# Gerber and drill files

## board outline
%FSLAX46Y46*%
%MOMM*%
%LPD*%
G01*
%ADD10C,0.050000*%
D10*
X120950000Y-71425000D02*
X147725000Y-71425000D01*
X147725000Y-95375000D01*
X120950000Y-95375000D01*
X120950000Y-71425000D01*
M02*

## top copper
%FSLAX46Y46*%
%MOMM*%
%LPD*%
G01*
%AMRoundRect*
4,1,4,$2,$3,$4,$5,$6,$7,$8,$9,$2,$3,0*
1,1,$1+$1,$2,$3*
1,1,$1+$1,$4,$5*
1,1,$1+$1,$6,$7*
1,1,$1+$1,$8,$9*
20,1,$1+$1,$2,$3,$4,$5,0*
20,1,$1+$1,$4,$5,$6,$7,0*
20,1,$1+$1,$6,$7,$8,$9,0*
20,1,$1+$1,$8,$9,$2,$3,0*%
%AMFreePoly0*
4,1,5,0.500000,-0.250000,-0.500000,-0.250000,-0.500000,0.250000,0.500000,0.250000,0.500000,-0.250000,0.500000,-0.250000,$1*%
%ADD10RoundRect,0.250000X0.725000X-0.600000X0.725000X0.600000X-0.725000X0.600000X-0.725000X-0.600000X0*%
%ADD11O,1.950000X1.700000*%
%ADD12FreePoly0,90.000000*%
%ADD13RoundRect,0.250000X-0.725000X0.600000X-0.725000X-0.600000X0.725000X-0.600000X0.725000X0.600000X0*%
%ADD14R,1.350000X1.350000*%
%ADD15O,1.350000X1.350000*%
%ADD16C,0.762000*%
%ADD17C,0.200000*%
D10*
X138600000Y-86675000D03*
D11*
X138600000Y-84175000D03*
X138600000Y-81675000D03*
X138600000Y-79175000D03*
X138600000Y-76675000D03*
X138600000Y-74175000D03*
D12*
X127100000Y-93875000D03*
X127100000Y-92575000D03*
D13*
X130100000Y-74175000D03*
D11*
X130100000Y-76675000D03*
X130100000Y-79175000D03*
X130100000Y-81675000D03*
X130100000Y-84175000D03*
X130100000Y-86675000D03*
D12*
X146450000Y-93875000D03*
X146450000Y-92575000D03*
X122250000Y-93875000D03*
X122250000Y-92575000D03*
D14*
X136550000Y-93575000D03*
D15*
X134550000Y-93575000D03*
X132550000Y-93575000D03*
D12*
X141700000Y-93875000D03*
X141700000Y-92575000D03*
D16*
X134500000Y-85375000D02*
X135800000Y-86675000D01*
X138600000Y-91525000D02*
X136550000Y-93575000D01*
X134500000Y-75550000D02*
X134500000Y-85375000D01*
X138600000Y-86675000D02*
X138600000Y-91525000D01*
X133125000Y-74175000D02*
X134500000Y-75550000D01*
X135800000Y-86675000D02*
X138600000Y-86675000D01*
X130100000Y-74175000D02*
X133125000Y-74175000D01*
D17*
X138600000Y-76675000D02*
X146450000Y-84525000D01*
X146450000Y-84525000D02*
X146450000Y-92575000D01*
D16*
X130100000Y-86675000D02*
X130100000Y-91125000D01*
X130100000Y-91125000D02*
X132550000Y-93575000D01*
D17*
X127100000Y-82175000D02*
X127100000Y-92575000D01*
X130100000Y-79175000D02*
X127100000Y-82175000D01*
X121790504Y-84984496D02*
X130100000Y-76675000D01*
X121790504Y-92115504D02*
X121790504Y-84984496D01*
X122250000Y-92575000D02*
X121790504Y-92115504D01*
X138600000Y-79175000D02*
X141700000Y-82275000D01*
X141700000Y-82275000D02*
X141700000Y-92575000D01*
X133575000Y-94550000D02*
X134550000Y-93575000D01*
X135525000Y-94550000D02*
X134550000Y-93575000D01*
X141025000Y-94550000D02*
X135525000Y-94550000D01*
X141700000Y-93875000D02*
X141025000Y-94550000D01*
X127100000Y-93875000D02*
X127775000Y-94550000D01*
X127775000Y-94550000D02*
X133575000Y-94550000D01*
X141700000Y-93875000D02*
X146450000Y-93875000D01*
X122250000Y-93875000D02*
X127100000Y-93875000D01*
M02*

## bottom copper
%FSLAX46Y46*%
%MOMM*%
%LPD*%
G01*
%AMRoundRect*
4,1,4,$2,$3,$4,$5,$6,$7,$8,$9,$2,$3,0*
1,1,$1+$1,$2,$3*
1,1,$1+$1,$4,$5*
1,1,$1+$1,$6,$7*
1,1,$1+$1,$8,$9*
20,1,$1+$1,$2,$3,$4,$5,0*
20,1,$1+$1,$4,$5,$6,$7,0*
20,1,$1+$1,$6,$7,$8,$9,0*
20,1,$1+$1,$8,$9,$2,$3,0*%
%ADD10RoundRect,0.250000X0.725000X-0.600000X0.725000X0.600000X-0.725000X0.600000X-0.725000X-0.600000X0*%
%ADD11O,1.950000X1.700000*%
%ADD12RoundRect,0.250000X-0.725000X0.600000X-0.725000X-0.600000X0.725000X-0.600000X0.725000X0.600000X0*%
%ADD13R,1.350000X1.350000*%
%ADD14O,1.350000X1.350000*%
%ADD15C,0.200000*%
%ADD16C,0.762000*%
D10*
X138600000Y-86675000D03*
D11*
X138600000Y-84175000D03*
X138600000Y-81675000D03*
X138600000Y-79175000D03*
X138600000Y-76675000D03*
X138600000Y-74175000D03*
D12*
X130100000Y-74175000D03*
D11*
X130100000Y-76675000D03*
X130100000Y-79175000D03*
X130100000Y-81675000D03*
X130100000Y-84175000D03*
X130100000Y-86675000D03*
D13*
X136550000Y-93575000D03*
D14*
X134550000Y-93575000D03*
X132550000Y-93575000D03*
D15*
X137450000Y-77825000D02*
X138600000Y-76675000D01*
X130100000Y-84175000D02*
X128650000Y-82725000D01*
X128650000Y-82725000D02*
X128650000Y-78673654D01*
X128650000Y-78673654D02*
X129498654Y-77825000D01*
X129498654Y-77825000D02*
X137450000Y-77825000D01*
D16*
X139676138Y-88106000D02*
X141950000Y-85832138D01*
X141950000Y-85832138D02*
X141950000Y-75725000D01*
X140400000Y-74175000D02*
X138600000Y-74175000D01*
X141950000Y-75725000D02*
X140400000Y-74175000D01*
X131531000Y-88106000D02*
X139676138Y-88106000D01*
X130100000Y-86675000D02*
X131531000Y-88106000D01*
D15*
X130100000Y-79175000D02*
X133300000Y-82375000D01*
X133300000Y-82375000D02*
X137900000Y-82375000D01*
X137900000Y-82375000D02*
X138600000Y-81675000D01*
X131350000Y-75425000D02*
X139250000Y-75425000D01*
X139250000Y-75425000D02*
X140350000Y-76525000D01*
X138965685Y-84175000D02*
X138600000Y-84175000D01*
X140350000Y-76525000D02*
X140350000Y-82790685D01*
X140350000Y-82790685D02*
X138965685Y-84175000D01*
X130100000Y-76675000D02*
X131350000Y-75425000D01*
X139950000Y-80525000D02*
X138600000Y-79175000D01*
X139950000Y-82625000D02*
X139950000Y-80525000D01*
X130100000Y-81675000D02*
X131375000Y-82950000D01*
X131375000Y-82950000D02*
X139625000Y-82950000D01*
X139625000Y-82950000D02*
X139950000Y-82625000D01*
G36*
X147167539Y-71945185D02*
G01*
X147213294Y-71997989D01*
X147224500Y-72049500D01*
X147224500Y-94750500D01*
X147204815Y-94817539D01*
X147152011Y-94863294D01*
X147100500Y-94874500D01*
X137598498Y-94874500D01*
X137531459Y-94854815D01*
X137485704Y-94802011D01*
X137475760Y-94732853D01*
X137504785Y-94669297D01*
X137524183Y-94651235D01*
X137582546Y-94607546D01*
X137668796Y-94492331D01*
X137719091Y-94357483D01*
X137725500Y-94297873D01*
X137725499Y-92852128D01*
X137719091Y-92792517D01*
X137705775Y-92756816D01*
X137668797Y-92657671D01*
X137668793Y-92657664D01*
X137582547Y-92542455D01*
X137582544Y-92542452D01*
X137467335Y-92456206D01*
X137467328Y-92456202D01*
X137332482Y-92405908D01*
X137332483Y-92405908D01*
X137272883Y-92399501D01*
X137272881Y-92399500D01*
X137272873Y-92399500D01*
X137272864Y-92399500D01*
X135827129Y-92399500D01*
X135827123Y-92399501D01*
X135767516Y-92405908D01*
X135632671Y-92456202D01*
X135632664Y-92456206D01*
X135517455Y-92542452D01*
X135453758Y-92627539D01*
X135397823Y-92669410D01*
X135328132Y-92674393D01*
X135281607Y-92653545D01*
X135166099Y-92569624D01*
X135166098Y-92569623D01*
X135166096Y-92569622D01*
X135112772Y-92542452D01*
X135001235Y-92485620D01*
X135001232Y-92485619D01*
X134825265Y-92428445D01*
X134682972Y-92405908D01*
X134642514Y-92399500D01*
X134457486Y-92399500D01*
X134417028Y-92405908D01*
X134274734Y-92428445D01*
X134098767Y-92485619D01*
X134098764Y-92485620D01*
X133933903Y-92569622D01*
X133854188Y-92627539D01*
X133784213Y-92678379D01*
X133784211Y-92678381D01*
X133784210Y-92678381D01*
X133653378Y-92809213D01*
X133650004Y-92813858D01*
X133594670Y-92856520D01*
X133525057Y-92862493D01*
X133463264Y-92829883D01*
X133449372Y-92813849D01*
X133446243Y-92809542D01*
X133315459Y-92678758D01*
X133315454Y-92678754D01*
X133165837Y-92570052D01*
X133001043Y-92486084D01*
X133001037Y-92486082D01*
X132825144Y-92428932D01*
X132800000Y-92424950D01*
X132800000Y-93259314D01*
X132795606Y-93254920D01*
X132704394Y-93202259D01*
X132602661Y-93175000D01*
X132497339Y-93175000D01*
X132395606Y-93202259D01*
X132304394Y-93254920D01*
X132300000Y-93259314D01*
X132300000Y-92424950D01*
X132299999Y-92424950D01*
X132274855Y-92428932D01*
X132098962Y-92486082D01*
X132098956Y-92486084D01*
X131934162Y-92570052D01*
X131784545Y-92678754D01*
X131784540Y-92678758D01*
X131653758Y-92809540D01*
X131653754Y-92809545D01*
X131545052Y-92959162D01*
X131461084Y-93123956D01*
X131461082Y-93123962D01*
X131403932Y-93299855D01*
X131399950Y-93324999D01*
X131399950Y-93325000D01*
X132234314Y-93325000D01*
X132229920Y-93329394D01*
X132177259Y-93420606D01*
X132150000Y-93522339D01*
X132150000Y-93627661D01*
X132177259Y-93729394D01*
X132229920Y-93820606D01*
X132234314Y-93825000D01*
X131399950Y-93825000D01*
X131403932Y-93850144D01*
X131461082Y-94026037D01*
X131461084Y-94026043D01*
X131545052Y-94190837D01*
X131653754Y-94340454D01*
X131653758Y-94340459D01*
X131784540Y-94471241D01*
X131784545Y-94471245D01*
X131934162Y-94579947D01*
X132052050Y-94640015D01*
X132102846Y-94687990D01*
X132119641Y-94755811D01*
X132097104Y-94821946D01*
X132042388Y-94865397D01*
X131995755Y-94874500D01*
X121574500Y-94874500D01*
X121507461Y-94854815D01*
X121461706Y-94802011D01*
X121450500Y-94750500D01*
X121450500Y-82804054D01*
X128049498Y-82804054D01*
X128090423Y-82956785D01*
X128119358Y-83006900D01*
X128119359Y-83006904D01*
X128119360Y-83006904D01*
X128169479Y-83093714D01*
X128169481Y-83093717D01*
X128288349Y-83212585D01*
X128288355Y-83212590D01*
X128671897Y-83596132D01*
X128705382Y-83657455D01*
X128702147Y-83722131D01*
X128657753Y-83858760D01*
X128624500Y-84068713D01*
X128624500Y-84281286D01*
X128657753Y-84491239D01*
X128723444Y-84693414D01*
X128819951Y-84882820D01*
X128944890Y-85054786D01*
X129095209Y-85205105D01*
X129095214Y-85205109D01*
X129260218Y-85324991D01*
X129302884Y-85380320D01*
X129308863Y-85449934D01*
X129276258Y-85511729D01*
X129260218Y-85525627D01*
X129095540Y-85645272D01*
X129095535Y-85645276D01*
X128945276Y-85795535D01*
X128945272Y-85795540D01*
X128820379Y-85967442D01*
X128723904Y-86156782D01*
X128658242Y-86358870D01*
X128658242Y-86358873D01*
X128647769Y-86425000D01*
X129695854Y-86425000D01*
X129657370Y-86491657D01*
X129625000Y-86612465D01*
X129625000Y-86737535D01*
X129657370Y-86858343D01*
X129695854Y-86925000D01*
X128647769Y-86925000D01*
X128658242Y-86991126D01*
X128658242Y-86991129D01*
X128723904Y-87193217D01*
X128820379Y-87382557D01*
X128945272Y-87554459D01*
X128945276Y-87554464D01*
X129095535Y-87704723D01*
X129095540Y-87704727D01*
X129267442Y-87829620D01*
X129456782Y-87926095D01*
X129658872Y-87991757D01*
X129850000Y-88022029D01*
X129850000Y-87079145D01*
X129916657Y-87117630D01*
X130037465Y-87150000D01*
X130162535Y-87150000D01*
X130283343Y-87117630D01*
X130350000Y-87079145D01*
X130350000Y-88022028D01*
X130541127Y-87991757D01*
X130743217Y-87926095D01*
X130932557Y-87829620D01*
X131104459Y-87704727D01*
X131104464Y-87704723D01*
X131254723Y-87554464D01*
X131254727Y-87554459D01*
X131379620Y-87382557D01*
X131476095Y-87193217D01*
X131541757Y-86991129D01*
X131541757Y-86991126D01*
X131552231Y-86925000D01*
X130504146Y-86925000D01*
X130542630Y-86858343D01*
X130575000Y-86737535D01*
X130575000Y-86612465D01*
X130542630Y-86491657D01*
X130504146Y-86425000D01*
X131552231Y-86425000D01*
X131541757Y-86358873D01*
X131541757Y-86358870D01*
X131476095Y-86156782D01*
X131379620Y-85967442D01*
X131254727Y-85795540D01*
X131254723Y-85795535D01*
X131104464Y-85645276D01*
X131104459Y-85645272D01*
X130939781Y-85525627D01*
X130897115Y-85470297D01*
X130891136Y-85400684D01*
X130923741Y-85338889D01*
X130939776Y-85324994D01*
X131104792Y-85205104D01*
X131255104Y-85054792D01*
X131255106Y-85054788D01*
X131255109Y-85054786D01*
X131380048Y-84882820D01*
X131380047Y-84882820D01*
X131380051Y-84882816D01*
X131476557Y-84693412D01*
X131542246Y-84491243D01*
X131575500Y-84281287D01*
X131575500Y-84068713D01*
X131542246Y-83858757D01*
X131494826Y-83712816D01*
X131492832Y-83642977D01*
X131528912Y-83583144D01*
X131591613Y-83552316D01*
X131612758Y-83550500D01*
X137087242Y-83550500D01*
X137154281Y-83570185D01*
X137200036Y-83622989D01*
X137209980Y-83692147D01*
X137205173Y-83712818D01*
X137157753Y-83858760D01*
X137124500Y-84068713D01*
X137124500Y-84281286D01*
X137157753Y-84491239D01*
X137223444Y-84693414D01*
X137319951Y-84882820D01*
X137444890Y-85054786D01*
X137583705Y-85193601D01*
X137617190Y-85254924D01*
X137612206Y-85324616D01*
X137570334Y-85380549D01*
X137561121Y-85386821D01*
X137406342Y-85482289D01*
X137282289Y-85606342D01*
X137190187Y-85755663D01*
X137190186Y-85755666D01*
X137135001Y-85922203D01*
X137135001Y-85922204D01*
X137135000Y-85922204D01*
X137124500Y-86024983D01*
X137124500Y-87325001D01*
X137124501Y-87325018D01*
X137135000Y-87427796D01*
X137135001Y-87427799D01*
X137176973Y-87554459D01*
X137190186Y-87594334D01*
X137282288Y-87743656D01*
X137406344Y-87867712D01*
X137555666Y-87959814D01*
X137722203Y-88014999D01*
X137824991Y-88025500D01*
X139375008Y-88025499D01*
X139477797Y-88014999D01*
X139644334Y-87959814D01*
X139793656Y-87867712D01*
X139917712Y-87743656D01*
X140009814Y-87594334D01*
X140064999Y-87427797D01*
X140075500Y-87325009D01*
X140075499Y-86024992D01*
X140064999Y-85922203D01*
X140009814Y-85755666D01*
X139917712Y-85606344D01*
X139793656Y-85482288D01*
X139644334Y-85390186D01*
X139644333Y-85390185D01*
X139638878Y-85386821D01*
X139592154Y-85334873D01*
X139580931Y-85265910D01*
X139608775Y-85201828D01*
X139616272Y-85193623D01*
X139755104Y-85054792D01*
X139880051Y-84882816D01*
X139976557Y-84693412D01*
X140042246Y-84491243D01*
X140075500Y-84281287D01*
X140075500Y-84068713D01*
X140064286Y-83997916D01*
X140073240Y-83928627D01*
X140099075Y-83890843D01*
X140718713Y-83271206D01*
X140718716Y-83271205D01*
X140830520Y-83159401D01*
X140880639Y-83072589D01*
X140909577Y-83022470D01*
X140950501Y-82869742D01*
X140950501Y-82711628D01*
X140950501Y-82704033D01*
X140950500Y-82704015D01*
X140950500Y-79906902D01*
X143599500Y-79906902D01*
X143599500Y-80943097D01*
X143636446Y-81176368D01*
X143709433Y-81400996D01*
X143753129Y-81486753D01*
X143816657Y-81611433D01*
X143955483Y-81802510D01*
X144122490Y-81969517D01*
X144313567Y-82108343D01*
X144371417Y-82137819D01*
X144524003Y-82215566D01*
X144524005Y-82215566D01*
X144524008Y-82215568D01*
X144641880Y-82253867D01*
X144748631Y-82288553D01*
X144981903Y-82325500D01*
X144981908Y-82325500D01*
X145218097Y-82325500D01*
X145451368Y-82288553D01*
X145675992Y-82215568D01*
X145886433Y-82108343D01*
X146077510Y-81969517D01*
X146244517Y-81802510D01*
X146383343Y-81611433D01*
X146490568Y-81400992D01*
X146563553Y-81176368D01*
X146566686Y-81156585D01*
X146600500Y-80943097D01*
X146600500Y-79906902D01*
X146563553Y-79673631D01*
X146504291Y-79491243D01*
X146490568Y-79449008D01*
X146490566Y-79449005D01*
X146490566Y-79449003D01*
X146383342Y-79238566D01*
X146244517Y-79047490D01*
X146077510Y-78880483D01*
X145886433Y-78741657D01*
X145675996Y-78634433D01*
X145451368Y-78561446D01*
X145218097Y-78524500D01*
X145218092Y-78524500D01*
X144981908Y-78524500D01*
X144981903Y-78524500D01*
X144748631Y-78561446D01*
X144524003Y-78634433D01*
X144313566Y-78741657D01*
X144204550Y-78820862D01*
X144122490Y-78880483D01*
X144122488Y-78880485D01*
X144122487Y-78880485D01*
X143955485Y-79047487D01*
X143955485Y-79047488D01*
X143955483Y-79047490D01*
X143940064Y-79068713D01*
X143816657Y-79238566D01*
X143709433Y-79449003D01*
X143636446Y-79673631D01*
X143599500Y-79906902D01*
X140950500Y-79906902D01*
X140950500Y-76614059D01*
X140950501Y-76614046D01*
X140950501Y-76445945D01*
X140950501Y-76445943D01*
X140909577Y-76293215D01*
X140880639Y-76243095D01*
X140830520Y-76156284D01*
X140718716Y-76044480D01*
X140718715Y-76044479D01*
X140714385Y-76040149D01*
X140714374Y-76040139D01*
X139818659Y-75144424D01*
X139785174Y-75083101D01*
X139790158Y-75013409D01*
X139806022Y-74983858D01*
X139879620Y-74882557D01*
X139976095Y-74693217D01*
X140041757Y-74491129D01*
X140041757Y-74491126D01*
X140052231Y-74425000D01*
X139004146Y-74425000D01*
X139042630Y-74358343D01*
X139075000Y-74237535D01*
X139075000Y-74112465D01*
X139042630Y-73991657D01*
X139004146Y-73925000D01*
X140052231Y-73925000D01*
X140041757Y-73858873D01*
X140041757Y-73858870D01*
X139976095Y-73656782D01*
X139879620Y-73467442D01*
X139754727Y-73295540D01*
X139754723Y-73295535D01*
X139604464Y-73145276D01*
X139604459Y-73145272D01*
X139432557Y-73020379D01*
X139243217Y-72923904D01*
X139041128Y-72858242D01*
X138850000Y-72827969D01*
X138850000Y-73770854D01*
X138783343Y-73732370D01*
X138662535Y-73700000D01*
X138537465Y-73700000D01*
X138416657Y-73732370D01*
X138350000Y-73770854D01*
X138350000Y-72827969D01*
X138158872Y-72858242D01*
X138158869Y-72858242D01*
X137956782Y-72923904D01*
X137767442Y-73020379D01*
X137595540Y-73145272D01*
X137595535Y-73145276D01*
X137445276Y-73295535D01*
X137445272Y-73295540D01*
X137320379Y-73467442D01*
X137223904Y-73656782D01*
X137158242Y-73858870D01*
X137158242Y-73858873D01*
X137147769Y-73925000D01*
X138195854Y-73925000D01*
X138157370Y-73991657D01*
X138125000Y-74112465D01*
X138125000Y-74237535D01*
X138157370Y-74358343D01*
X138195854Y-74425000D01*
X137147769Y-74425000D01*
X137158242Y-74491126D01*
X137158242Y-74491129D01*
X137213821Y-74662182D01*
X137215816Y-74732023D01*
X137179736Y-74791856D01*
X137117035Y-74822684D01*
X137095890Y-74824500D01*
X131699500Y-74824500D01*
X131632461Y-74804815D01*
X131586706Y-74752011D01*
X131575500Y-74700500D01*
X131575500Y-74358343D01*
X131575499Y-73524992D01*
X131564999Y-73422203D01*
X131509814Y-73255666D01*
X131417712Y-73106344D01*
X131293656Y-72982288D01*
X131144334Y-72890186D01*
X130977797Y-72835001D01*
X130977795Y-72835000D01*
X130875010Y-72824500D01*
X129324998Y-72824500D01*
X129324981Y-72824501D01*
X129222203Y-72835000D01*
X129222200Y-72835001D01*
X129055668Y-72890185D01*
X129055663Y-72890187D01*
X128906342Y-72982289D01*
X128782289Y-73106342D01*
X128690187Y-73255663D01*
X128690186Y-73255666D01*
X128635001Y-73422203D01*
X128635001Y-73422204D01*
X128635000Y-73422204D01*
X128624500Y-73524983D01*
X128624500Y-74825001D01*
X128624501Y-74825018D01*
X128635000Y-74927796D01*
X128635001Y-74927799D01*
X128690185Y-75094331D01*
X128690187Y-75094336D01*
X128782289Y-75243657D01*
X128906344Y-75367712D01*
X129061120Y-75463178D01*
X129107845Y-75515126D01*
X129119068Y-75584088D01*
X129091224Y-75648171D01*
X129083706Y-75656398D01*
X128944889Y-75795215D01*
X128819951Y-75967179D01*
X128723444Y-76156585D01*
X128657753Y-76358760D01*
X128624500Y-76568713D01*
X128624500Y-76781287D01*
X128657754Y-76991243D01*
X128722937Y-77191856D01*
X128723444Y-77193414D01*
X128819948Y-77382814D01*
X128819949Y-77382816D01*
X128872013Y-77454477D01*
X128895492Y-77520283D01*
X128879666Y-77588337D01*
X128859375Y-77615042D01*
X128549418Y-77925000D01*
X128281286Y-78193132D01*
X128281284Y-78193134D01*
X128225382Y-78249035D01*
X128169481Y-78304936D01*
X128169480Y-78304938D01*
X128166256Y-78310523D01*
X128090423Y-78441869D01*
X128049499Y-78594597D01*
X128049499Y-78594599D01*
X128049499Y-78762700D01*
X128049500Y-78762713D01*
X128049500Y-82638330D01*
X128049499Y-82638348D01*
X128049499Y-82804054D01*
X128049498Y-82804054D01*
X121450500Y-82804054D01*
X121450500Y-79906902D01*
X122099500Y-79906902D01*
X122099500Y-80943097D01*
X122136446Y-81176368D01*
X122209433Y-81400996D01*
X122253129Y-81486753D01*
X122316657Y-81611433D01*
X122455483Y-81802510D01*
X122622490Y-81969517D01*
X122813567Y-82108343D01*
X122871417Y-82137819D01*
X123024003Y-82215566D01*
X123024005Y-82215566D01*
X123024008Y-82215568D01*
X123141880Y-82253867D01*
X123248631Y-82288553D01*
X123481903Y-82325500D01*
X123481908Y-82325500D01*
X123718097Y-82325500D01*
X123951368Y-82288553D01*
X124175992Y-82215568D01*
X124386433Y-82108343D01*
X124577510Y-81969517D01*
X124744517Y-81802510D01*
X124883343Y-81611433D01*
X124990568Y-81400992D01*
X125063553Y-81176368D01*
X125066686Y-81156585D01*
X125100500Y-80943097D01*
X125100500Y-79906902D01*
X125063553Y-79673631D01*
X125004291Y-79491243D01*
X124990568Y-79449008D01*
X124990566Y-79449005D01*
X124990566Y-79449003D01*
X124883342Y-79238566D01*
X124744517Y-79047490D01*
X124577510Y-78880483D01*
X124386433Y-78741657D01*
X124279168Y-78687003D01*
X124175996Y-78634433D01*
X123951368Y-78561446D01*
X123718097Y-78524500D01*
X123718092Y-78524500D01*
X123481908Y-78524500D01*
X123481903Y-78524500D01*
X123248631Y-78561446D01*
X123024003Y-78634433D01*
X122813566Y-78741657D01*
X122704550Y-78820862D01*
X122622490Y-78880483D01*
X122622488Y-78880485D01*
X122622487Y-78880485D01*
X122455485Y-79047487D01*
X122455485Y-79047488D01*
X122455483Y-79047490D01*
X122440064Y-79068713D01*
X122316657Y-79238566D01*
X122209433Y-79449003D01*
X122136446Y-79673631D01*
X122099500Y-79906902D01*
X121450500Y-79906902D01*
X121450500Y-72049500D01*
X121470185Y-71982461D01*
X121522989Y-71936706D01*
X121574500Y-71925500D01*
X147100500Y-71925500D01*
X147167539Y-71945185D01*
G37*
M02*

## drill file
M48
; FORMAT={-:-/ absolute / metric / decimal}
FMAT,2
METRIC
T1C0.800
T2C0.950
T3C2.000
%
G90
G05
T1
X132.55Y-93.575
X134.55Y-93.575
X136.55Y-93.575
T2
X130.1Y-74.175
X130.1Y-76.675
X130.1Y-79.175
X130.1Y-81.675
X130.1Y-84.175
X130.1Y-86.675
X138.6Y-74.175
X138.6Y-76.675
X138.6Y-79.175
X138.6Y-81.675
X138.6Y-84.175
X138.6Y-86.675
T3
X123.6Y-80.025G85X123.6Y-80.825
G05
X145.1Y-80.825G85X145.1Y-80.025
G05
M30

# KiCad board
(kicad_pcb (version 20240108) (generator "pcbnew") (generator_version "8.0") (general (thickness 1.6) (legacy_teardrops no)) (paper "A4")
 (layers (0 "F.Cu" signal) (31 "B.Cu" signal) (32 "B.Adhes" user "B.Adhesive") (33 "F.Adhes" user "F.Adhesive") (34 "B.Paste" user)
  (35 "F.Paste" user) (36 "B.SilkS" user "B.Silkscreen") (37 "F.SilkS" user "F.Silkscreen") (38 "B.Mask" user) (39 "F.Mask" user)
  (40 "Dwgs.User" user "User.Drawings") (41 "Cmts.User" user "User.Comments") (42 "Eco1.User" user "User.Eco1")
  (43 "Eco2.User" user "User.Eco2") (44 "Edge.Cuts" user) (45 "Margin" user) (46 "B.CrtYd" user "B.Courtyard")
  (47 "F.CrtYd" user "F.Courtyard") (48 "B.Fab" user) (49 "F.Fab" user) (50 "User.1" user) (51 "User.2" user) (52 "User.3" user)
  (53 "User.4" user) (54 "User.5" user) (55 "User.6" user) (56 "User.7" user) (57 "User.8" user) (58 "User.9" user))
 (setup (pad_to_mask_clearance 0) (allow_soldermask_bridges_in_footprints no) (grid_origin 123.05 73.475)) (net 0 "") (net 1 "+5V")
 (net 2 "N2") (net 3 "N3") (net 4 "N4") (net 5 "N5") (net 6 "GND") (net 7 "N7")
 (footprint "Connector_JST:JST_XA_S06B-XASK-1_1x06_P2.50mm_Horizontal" (layer "F.Cu") (at 138.6 86.675 90)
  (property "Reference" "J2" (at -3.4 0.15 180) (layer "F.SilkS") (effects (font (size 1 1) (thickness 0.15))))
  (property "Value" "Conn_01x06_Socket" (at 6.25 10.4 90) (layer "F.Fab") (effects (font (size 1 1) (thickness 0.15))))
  (pad "" np_thru_hole oval (at 6.25 6.5 90) (size 2.8 2) (drill oval 2.8 2) (layers "*.Cu" "*.Mask"))
  (pad "1" thru_hole roundrect (at 0 0 90) (size 1.7 1.95) (drill 0.95) (layers "*.Cu" "*.Mask") (remove_unused_layers no)
   (roundrect_rratio 0.1470588235) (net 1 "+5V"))
  (pad "2" thru_hole oval (at 2.5 0 90) (size 1.7 1.95) (drill 0.95) (layers "*.Cu" "*.Mask") (remove_unused_layers no) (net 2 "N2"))
  (pad "3" thru_hole oval (at 5 0 90) (size 1.7 1.95) (drill 0.95) (layers "*.Cu" "*.Mask") (remove_unused_layers no) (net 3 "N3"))
  (pad "4" thru_hole oval (at 7.5 0 90) (size 1.7 1.95) (drill 0.95) (layers "*.Cu" "*.Mask") (remove_unused_layers no) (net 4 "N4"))
  (pad "5" thru_hole oval (at 10 0 90) (size 1.7 1.95) (drill 0.95) (layers "*.Cu" "*.Mask") (remove_unused_layers no) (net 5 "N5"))
  (pad "6" thru_hole oval (at 12.5 0 90) (size 1.7 1.95) (drill 0.95) (layers "*.Cu" "*.Mask") (remove_unused_layers no) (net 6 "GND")))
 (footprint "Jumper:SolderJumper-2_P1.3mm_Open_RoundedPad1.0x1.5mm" (layer "F.Cu") (at 127.1 93.225 90)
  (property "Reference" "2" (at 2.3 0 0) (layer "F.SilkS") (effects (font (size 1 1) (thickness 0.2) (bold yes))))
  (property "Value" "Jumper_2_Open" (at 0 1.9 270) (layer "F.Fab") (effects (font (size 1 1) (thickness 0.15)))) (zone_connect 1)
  (pad "1" smd custom (at -0.65 0 90) (size 1 0.5) (layers "F.Cu" "F.Mask") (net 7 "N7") (zone_connect 2) (thermal_bridge_angle 45)
   (options (clearance outline) (anchor rect)) (primitives))
  (pad "2" smd custom (at 0.65 0 90) (size 1 0.5) (layers "F.Cu" "F.Mask") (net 3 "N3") (zone_connect 2) (thermal_bridge_angle 45)
   (options (clearance outline) (anchor rect)) (primitives)))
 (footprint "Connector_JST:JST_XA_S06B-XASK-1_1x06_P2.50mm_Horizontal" (layer "F.Cu") (at 130.1 74.175 -90)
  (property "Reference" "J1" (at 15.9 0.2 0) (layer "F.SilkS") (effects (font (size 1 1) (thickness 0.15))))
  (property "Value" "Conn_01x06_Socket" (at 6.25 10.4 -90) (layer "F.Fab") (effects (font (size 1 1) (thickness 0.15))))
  (pad "" np_thru_hole oval (at 6.25 6.5 270) (size 2.8 2) (drill oval 2.8 2) (layers "*.Cu" "*.Mask"))
  (pad "1" thru_hole roundrect (at 0 0 270) (size 1.7 1.95) (drill 0.95) (layers "*.Cu" "*.Mask") (remove_unused_layers no)
   (roundrect_rratio 0.1470588235) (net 1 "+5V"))
  (pad "2" thru_hole oval (at 2.5 0 270) (size 1.7 1.95) (drill 0.95) (layers "*.Cu" "*.Mask") (remove_unused_layers no) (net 2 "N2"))
  (pad "3" thru_hole oval (at 5 0 270) (size 1.7 1.95) (drill 0.95) (layers "*.Cu" "*.Mask") (remove_unused_layers no) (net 3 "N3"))
  (pad "4" thru_hole oval (at 7.5 0 270) (size 1.7 1.95) (drill 0.95) (layers "*.Cu" "*.Mask") (remove_unused_layers no) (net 4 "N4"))
  (pad "5" thru_hole oval (at 10 0 270) (size 1.7 1.95) (drill 0.95) (layers "*.Cu" "*.Mask") (remove_unused_layers no) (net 5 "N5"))
  (pad "6" thru_hole oval (at 12.5 0 270) (size 1.7 1.95) (drill 0.95) (layers "*.Cu" "*.Mask") (remove_unused_layers no) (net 6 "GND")))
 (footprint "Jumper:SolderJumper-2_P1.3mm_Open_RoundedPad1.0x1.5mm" (layer "F.Cu") (at 146.45 93.225 90)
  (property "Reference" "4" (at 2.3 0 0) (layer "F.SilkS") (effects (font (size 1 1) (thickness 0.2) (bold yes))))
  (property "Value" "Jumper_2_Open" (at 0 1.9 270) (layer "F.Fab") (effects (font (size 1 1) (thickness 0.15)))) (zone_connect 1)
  (pad "1" smd custom (at -0.65 0 90) (size 1 0.5) (layers "F.Cu" "F.Mask") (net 7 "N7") (zone_connect 2) (thermal_bridge_angle 45)
   (options (clearance outline) (anchor rect)) (primitives))
  (pad "2" smd custom (at 0.65 0 90) (size 1 0.5) (layers "F.Cu" "F.Mask") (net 5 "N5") (zone_connect 2) (thermal_bridge_angle 45)
   (options (clearance outline) (anchor rect)) (primitives)))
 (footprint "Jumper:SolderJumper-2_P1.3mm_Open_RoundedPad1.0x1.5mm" (layer "F.Cu") (at 122.25 93.225 90)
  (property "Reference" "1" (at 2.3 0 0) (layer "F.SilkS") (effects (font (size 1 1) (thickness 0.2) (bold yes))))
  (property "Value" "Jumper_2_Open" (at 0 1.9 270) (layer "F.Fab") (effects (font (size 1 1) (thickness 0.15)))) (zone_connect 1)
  (pad "1" smd custom (at -0.65 0 90) (size 1 0.5) (layers "F.Cu" "F.Mask") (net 7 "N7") (zone_connect 2) (thermal_bridge_angle 45)
   (options (clearance outline) (anchor rect)) (primitives))
  (pad "2" smd custom (at 0.65 0 90) (size 1 0.5) (layers "F.Cu" "F.Mask") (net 2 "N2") (zone_connect 2) (thermal_bridge_angle 45)
   (options (clearance outline) (anchor rect)) (primitives)))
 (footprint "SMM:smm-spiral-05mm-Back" (layer "F.Cu") (at 134.6 79.675)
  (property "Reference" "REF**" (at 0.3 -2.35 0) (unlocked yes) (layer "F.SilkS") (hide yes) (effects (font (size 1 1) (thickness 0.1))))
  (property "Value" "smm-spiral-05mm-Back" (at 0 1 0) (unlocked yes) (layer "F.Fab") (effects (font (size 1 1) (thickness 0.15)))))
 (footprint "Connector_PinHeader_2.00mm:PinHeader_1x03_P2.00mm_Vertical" (layer "F.Cu") (at 136.55 93.575 -90)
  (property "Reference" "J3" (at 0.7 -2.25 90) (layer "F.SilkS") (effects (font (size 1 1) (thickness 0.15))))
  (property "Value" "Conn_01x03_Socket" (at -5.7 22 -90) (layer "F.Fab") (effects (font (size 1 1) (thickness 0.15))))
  (pad "1" thru_hole rect (at 0 0 270) (size 1.35 1.35) (drill 0.8) (layers "*.Cu" "*.Mask") (remove_unused_layers no) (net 1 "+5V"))
  (pad "2" thru_hole oval (at 0 2 270) (size 1.35 1.35) (drill 0.8) (layers "*.Cu" "*.Mask") (remove_unused_layers no) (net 7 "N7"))
  (pad "3" thru_hole oval (at 0 4 270) (size 1.35 1.35) (drill 0.8) (layers "*.Cu" "*.Mask") (remove_unused_layers no) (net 6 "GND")))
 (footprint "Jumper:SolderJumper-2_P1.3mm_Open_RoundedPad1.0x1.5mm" (layer "F.Cu") (at 141.7 93.225 90)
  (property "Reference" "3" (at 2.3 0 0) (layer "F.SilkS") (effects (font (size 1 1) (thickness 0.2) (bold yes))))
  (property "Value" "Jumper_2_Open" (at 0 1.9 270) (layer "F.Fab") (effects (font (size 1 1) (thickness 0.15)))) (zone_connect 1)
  (pad "1" smd custom (at -0.65 0 90) (size 1 0.5) (layers "F.Cu" "F.Mask") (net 7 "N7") (zone_connect 2) (thermal_bridge_angle 45)
   (options (clearance outline) (anchor rect)) (primitives))
  (pad "2" smd custom (at 0.65 0 90) (size 1 0.5) (layers "F.Cu" "F.Mask") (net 4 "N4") (zone_connect 2) (thermal_bridge_angle 45)
   (options (clearance outline) (anchor rect)) (primitives)))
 (gr_rect (start 120.95 71.425) (end 147.725 95.375) (stroke (width 0.05) (type default)) (fill none) (layer "Edge.Cuts"))
 (segment (start 134.5 85.375) (end 135.8 86.675) (width 0.762) (layer "F.Cu") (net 1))
 (segment (start 138.6 91.525) (end 136.55 93.575) (width 0.762) (layer "F.Cu") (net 1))
 (segment (start 134.5 75.55) (end 134.5 85.375) (width 0.762) (layer "F.Cu") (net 1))
 (segment (start 138.6 86.675) (end 138.6 91.525) (width 0.762) (layer "F.Cu") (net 1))
 (segment (start 133.125 74.175) (end 134.5 75.55) (width 0.762) (layer "F.Cu") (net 1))
 (segment (start 135.8 86.675) (end 138.6 86.675) (width 0.762) (layer "F.Cu") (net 1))
 (segment (start 130.1 74.175) (end 133.125 74.175) (width 0.762) (layer "F.Cu") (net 1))
 (segment (start 138.6 76.675) (end 146.45 84.525) (width 0.2) (layer "F.Cu") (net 5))
 (segment (start 146.45 84.525) (end 146.45 92.575) (width 0.2) (layer "F.Cu") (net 5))
 (segment (start 137.45 77.825) (end 138.6 76.675) (width 0.2) (layer "B.Cu") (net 5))
 (segment (start 130.1 84.175) (end 128.65 82.725) (width 0.2) (layer "B.Cu") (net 5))
 (segment (start 128.65 82.725) (end 128.65 78.673654) (width 0.2) (layer "B.Cu") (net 5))
 (segment (start 128.65 78.673654) (end 129.498654 77.825) (width 0.2) (layer "B.Cu") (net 5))
 (segment (start 129.498654 77.825) (end 137.45 77.825) (width 0.2) (layer "B.Cu") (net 5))
 (segment (start 130.1 86.675) (end 130.1 91.125) (width 0.762) (layer "F.Cu") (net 6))
 (segment (start 130.1 91.125) (end 132.55 93.575) (width 0.762) (layer "F.Cu") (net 6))
 (segment (start 139.676138 88.106) (end 141.95 85.832138) (width 0.762) (layer "B.Cu") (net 6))
 (segment (start 141.95 85.832138) (end 141.95 75.725) (width 0.762) (layer "B.Cu") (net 6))
 (segment (start 140.4 74.175) (end 138.6 74.175) (width 0.762) (layer "B.Cu") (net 6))
 (segment (start 141.95 75.725) (end 140.4 74.175) (width 0.762) (layer "B.Cu") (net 6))
 (segment (start 131.531 88.106) (end 139.676138 88.106) (width 0.762) (layer "B.Cu") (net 6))
 (segment (start 130.1 86.675) (end 131.531 88.106) (width 0.762) (layer "B.Cu") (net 6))
 (segment (start 127.1 82.175) (end 127.1 92.575) (width 0.2) (layer "F.Cu") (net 3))
 (segment (start 130.1 79.175) (end 127.1 82.175) (width 0.2) (layer "F.Cu") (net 3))
 (segment (start 130.1 79.175) (end 133.3 82.375) (width 0.2) (layer "B.Cu") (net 3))
 (segment (start 133.3 82.375) (end 137.9 82.375) (width 0.2) (layer "B.Cu") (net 3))
 (segment (start 137.9 82.375) (end 138.6 81.675) (width 0.2) (layer "B.Cu") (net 3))
 (segment (start 121.790504 84.984496) (end 130.1 76.675) (width 0.2) (layer "F.Cu") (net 2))
 (segment (start 121.790504 92.115504) (end 121.790504 84.984496) (width 0.2) (layer "F.Cu") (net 2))
 (segment (start 122.25 92.575) (end 121.790504 92.115504) (width 0.2) (layer "F.Cu") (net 2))
 (segment (start 131.35 75.425) (end 139.25 75.425) (width 0.2) (layer "B.Cu") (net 2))
 (segment (start 139.25 75.425) (end 140.35 76.525) (width 0.2) (layer "B.Cu") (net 2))
 (segment (start 138.965685 84.175) (end 138.6 84.175) (width 0.2) (layer "B.Cu") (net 2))
 (segment (start 140.35 76.525) (end 140.35 82.790685) (width 0.2) (layer "B.Cu") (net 2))
 (segment (start 140.35 82.790685) (end 138.965685 84.175) (width 0.2) (layer "B.Cu") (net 2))
 (segment (start 130.1 76.675) (end 131.35 75.425) (width 0.2) (layer "B.Cu") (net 2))
 (segment (start 138.6 79.175) (end 141.7 82.275) (width 0.2) (layer "F.Cu") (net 4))
 (segment (start 141.7 82.275) (end 141.7 92.575) (width 0.2) (layer "F.Cu") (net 4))
 (segment (start 139.95 80.525) (end 138.6 79.175) (width 0.2) (layer "B.Cu") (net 4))
 (segment (start 139.95 82.625) (end 139.95 80.525) (width 0.2) (layer "B.Cu") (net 4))
 (segment (start 130.1 81.675) (end 131.375 82.95) (width 0.2) (layer "B.Cu") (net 4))
 (segment (start 131.375 82.95) (end 139.625 82.95) (width 0.2) (layer "B.Cu") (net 4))
 (segment (start 139.625 82.95) (end 139.95 82.625) (width 0.2) (layer "B.Cu") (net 4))
 (segment (start 133.575 94.55) (end 134.55 93.575) (width 0.2) (layer "F.Cu") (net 7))
 (segment (start 135.525 94.55) (end 134.55 93.575) (width 0.2) (layer "F.Cu") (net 7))
 (segment (start 141.025 94.55) (end 135.525 94.55) (width 0.2) (layer "F.Cu") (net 7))
 (segment (start 141.7 93.875) (end 141.025 94.55) (width 0.2) (layer "F.Cu") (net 7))
 (segment (start 127.1 93.875) (end 127.775 94.55) (width 0.2) (layer "F.Cu") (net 7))
 (segment (start 127.775 94.55) (end 133.575 94.55) (width 0.2) (layer "F.Cu") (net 7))
 (segment (start 141.7 93.875) (end 146.45 93.875) (width 0.2) (layer "F.Cu") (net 7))
 (segment (start 122.25 93.875) (end 127.1 93.875) (width 0.2) (layer "F.Cu") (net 7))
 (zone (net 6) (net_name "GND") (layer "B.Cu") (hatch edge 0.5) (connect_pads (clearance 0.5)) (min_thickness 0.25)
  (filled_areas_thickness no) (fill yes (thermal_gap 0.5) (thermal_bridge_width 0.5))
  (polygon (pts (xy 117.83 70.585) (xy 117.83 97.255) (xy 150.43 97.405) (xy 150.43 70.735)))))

